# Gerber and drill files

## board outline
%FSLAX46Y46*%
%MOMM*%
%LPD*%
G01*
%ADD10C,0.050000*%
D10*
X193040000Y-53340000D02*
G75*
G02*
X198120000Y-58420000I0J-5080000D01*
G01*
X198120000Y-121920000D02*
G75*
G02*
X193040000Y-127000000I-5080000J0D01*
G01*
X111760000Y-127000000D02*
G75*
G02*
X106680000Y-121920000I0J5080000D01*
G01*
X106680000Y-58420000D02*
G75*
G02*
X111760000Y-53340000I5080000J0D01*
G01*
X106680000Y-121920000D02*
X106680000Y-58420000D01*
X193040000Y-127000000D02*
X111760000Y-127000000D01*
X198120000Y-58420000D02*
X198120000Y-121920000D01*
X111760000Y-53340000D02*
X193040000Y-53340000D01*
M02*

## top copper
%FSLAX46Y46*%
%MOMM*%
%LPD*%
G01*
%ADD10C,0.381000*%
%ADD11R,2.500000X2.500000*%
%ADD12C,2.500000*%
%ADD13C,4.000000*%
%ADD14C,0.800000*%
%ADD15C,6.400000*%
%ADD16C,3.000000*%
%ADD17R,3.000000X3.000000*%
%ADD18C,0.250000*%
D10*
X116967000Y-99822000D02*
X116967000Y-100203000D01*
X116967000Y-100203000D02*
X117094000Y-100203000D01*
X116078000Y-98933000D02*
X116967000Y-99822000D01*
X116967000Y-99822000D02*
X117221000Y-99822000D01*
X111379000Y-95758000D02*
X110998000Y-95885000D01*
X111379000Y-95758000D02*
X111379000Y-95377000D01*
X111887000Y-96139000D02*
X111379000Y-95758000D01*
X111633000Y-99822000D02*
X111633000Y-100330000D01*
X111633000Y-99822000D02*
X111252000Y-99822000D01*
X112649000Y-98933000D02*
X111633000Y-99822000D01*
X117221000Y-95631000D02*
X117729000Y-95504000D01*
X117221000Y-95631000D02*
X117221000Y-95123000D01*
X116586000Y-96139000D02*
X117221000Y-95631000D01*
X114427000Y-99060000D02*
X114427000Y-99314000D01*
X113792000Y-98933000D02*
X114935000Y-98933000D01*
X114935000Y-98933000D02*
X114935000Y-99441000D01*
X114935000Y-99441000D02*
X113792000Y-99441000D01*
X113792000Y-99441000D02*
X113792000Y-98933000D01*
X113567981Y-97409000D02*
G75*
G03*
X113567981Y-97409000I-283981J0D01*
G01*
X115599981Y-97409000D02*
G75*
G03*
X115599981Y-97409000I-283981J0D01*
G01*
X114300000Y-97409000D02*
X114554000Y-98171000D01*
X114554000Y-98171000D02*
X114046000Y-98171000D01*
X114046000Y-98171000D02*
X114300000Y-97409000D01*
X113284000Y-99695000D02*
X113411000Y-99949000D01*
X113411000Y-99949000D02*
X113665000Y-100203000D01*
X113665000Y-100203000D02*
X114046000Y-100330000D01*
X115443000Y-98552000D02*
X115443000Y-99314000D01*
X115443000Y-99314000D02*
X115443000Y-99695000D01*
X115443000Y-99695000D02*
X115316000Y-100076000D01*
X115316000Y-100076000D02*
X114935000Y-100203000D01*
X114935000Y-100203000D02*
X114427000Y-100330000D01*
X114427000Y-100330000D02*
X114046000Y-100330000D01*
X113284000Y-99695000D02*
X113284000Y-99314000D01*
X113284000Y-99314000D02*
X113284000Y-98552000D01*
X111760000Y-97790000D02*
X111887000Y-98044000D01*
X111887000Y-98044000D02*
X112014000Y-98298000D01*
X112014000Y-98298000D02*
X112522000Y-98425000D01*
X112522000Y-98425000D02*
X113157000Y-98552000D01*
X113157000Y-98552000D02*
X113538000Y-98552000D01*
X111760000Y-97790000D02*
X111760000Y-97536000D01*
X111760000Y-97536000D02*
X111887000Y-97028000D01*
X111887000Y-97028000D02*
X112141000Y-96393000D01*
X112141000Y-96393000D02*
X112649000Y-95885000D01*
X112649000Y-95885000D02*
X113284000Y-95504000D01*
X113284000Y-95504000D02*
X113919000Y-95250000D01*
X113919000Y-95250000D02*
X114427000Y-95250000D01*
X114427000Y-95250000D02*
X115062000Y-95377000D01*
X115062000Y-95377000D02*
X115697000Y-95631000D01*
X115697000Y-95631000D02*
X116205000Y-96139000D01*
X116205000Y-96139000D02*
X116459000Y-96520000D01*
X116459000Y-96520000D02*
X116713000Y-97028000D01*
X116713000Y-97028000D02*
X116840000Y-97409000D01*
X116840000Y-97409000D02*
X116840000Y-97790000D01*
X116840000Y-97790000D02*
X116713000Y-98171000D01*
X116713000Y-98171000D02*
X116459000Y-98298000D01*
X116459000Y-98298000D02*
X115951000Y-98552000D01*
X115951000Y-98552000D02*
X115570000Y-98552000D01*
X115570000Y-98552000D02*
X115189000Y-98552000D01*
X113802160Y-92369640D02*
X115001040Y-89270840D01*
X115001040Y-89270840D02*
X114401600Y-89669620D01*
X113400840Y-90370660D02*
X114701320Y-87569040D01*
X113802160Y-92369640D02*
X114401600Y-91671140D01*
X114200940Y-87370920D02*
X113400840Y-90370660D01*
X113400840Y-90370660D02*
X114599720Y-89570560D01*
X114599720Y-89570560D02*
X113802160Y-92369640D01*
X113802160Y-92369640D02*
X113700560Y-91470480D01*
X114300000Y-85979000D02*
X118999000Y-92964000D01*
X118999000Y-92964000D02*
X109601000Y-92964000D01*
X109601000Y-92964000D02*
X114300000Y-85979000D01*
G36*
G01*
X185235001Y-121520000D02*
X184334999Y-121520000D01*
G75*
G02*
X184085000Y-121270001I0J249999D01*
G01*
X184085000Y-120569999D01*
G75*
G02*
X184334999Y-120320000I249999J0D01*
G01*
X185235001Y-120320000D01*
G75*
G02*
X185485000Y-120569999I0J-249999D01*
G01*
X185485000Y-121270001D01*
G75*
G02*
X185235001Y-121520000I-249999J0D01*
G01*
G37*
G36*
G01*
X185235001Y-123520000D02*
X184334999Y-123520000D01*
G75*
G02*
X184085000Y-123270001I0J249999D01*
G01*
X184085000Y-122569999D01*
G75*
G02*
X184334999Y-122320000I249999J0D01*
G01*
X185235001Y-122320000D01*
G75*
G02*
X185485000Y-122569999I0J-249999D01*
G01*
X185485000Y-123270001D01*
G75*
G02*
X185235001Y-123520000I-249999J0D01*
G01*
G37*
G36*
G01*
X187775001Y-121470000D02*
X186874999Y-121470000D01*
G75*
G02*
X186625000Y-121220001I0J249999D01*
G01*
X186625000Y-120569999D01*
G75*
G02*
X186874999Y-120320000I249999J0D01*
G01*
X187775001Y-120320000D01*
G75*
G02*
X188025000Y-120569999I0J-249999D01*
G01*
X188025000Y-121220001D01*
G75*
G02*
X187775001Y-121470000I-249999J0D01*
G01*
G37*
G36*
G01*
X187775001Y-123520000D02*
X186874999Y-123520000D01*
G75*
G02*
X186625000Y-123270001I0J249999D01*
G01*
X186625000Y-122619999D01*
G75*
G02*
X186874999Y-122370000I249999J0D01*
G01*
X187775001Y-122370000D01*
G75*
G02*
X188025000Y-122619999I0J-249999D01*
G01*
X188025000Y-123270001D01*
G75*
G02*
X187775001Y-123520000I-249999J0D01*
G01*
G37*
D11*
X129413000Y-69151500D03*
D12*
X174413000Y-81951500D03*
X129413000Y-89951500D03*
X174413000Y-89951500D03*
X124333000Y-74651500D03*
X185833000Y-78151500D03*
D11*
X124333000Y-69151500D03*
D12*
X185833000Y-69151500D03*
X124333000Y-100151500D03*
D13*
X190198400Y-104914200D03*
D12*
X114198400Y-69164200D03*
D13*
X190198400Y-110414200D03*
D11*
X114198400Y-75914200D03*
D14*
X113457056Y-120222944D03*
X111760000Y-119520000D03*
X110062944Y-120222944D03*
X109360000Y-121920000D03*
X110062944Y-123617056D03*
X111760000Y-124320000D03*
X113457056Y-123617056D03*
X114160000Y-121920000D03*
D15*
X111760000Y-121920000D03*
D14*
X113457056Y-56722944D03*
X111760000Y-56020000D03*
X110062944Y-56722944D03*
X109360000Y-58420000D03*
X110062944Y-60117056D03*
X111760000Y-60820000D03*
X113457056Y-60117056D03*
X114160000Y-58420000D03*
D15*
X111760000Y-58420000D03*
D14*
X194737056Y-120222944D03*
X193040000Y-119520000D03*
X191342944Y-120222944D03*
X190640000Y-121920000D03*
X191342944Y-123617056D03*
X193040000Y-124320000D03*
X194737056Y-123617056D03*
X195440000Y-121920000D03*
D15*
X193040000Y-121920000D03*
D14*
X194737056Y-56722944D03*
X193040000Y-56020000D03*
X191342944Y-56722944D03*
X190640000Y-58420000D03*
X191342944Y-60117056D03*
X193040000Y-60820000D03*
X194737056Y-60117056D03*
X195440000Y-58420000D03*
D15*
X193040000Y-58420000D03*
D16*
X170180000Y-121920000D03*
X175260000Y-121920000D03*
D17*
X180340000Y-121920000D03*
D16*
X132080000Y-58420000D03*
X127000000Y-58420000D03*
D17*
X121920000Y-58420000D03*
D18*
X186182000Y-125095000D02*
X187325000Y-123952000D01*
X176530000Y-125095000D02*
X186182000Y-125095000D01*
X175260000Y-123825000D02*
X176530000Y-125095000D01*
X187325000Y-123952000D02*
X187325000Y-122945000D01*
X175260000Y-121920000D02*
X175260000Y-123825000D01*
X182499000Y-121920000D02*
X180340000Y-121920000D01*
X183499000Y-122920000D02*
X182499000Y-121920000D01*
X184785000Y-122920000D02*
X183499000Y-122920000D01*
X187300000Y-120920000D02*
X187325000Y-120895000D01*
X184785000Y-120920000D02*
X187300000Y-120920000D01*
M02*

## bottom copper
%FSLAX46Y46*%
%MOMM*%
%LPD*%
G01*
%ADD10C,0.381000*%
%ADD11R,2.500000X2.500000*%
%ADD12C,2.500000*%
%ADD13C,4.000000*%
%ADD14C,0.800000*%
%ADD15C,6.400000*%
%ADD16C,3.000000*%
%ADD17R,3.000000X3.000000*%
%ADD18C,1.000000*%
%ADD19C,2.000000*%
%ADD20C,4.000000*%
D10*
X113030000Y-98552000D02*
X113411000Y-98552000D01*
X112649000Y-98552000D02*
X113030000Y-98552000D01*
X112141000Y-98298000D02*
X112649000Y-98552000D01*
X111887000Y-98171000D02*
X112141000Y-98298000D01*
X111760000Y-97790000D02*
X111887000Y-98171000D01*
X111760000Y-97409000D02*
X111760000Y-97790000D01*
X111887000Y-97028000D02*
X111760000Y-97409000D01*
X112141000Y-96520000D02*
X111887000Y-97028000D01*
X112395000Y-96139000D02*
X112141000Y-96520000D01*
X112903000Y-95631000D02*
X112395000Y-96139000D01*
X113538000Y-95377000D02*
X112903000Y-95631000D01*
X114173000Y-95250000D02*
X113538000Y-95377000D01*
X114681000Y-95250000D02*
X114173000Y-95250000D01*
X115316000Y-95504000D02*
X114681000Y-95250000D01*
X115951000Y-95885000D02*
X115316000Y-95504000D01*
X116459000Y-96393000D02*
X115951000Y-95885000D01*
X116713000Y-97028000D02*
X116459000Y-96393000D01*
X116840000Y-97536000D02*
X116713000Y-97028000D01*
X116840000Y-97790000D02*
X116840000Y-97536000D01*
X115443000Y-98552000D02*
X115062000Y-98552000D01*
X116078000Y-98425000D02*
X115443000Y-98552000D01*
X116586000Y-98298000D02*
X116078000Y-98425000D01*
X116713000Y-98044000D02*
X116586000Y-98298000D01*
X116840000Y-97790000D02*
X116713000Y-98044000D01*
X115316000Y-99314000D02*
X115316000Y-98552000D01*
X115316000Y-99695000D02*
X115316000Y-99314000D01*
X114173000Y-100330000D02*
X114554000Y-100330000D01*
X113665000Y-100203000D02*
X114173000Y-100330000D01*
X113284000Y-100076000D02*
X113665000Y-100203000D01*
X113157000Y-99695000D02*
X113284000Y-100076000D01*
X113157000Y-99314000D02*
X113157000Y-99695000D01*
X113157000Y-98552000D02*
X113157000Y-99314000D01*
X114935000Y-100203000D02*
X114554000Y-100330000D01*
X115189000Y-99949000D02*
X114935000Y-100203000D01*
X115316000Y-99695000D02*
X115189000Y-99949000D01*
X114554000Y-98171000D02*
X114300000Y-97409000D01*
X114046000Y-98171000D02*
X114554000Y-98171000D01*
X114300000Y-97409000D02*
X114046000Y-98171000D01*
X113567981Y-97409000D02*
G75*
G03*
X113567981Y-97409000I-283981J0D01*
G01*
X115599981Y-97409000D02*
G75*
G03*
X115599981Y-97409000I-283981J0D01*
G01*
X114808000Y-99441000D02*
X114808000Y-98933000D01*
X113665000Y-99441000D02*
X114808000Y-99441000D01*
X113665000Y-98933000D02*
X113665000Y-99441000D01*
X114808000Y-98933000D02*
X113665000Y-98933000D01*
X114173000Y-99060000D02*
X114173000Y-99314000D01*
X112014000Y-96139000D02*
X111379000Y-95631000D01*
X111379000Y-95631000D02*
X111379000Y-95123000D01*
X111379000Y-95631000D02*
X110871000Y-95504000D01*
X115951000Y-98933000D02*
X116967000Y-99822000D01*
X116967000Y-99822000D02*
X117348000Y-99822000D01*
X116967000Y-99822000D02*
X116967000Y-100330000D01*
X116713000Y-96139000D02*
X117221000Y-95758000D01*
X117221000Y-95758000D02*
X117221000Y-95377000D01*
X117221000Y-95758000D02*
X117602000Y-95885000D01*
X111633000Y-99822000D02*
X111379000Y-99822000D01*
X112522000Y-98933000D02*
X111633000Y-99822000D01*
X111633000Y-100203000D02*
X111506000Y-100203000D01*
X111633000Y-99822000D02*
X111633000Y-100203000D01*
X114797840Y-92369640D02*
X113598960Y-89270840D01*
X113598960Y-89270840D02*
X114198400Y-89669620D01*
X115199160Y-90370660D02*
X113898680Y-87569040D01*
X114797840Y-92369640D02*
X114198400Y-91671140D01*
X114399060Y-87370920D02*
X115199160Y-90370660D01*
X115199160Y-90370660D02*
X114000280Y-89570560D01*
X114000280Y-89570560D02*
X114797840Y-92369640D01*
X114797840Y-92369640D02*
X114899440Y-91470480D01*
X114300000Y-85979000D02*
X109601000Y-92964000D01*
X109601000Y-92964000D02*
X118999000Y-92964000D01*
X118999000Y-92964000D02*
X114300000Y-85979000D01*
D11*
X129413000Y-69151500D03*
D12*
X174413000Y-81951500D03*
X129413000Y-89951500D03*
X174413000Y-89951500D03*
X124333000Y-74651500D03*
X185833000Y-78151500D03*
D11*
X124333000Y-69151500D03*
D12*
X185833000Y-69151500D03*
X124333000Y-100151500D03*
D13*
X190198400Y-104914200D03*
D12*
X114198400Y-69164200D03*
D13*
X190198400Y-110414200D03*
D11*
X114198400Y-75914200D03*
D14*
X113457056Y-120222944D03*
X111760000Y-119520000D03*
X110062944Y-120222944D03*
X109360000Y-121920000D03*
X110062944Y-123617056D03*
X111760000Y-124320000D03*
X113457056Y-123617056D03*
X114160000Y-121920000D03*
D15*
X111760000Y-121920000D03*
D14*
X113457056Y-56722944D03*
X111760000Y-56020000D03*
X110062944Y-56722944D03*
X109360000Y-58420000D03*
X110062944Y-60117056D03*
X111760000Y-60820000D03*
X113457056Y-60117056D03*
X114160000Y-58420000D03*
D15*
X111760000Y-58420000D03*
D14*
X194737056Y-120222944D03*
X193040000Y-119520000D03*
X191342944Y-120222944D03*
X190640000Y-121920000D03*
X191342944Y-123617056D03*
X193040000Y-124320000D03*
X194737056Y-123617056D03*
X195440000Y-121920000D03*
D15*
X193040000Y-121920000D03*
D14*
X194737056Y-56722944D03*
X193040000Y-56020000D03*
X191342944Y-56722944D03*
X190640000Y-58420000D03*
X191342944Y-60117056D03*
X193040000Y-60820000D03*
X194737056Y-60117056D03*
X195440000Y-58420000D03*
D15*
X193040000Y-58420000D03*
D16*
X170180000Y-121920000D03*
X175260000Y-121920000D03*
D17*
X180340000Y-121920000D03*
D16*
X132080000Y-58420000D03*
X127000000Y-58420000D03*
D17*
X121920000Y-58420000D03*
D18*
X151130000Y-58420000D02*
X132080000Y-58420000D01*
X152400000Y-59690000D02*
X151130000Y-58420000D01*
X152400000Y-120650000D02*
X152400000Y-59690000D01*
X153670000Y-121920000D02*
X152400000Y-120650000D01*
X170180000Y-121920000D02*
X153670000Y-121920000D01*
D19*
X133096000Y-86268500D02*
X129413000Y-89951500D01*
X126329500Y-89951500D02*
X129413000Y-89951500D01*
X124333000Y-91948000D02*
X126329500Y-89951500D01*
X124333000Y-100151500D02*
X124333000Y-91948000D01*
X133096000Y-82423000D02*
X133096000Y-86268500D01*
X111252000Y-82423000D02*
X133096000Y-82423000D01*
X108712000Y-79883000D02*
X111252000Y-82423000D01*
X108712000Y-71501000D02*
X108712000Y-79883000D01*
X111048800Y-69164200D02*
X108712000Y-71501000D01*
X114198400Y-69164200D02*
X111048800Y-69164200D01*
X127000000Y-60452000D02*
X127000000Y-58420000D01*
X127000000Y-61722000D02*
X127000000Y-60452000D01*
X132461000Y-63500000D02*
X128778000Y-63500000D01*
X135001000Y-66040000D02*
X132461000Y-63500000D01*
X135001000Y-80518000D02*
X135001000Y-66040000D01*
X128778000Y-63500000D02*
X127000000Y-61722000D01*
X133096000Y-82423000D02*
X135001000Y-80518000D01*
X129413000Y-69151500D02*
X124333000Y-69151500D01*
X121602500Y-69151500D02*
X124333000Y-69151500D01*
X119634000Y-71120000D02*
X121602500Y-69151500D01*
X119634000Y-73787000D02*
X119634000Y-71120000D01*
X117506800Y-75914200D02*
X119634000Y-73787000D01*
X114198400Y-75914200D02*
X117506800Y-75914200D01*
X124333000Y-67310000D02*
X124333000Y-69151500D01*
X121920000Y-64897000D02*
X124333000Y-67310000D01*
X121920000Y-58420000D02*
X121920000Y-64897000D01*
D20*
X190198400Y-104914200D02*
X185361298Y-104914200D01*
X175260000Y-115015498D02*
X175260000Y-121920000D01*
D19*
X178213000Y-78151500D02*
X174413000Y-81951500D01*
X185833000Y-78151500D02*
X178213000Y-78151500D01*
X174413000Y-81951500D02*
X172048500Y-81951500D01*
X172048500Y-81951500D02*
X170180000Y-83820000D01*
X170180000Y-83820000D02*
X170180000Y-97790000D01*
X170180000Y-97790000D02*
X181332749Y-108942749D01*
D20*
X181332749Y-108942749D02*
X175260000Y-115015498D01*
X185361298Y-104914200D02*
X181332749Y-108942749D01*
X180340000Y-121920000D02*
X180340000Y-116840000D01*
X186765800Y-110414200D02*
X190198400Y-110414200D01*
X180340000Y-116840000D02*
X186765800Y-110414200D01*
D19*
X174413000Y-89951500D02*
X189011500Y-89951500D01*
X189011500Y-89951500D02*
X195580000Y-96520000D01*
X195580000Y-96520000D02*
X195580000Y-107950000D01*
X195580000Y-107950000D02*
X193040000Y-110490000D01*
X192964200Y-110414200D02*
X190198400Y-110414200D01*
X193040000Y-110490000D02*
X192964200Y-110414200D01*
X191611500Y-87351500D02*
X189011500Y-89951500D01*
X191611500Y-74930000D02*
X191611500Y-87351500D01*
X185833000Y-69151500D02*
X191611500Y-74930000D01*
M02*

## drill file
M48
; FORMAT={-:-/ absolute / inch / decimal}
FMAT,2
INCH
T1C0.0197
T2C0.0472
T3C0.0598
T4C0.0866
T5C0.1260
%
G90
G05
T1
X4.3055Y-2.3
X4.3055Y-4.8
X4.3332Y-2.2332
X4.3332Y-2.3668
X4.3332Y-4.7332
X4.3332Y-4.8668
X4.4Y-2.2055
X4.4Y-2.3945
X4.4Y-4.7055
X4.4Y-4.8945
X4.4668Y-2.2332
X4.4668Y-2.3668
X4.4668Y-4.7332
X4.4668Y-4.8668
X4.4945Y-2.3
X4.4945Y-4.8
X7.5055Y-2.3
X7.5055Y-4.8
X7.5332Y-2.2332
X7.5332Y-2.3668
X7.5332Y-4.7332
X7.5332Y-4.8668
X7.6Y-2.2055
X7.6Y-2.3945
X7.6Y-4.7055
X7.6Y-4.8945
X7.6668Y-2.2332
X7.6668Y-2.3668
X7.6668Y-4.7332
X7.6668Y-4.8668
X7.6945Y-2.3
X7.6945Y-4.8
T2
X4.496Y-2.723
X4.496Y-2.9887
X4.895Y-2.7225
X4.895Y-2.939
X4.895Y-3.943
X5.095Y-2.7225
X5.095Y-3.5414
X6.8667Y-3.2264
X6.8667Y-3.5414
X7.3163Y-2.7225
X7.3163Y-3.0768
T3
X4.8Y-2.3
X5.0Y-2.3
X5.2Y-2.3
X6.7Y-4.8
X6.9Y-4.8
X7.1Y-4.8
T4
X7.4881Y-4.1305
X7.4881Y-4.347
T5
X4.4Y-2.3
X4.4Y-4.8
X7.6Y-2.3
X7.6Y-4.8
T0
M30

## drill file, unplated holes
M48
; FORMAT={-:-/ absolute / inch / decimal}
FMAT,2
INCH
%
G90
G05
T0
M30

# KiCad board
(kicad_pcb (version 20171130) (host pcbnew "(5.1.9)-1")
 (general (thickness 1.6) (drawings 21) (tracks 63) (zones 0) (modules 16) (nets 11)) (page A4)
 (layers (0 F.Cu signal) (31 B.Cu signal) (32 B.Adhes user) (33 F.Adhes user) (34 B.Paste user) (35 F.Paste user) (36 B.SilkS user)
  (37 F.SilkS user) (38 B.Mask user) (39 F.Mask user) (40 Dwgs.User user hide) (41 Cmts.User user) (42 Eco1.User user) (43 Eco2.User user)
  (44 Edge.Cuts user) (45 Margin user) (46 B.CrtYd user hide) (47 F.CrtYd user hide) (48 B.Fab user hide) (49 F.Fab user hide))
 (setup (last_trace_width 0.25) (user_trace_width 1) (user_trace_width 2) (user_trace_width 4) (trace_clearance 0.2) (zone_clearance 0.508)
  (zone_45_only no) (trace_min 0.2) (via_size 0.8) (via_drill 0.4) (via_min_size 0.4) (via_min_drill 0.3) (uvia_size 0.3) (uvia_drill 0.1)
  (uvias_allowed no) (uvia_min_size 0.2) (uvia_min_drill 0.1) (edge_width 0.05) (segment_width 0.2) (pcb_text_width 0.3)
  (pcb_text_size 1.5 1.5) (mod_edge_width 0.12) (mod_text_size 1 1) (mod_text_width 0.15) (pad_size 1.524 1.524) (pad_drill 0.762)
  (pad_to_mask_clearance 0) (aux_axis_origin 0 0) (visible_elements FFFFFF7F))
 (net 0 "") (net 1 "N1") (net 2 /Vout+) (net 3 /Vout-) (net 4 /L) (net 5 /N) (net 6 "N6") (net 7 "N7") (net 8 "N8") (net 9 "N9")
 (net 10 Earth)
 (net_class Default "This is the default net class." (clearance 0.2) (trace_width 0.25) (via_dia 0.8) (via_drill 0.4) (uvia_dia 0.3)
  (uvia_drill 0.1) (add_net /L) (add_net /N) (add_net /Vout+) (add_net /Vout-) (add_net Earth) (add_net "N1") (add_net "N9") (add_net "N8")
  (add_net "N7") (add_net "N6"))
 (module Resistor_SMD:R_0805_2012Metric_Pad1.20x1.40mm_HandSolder (layer F.Cu) (at 184.785 121.92 90)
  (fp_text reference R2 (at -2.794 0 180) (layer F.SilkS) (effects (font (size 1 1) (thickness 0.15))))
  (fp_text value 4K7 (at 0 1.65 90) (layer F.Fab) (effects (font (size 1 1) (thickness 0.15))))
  (pad 2 smd roundrect (at 1 0 90) (size 1.2 1.4) (layers F.Cu F.Paste F.Mask) (roundrect_rratio 0.2083325) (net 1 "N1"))
  (pad 1 smd roundrect (at -1 0 90) (size 1.2 1.4) (layers F.Cu F.Paste F.Mask) (roundrect_rratio 0.2083325) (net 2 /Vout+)))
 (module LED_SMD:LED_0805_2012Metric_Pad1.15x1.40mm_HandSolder (layer F.Cu) (at 187.325 121.92 90)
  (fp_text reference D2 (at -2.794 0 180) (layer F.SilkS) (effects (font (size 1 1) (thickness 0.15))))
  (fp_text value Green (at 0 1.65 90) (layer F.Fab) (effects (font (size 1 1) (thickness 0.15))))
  (pad 2 smd roundrect (at 1.025 0 90) (size 1.15 1.4) (layers F.Cu F.Paste F.Mask) (roundrect_rratio 0.2173904347826087) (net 1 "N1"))
  (pad 1 smd roundrect (at -1.025 0 90) (size 1.15 1.4) (layers F.Cu F.Paste F.Mask) (roundrect_rratio 0.2173904347826087) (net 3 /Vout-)))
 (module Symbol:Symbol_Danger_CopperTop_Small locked (layer B.Cu) (at 114.3 97.79 180)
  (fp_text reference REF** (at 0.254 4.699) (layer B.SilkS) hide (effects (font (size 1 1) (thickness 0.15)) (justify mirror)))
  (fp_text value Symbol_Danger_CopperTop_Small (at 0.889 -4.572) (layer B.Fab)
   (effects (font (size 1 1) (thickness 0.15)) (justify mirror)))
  (fp_line (start 1.27 -0.762) (end 0.889 -0.762) (layer B.Cu) (width 0.381))
  (fp_line (start 1.651 -0.762) (end 1.27 -0.762) (layer B.Cu) (width 0.381))
  (fp_line (start 2.159 -0.508) (end 1.651 -0.762) (layer B.Cu) (width 0.381))
  (fp_line (start 2.413 -0.381) (end 2.159 -0.508) (layer B.Cu) (width 0.381))
  (fp_line (start 2.54 0) (end 2.413 -0.381) (layer B.Cu) (width 0.381))
  (fp_line (start 2.54 0.381) (end 2.54 0) (layer B.Cu) (width 0.381))
  (fp_line (start 2.413 0.762) (end 2.54 0.381) (layer B.Cu) (width 0.381))
  (fp_line (start 2.159 1.27) (end 2.413 0.762) (layer B.Cu) (width 0.381))
  (fp_line (start 1.905 1.651) (end 2.159 1.27) (layer B.Cu) (width 0.381))
  (fp_line (start 1.397 2.159) (end 1.905 1.651) (layer B.Cu) (width 0.381))
  (fp_line (start 0.762 2.413) (end 1.397 2.159) (layer B.Cu) (width 0.381))
  (fp_line (start 0.127 2.54) (end 0.762 2.413) (layer B.Cu) (width 0.381))
  (fp_line (start -0.381 2.54) (end 0.127 2.54) (layer B.Cu) (width 0.381))
  (fp_line (start -1.016 2.286) (end -0.381 2.54) (layer B.Cu) (width 0.381))
  (fp_line (start -1.651 1.905) (end -1.016 2.286) (layer B.Cu) (width 0.381))
  (fp_line (start -2.159 1.397) (end -1.651 1.905) (layer B.Cu) (width 0.381))
  (fp_line (start -2.413 0.762) (end -2.159 1.397) (layer B.Cu) (width 0.381))
  (fp_line (start -2.54 0.254) (end -2.413 0.762) (layer B.Cu) (width 0.381))
  (fp_line (start -2.54 0) (end -2.54 0.254) (layer B.Cu) (width 0.381))
  (fp_line (start -1.143 -0.762) (end -0.762 -0.762) (layer B.Cu) (width 0.381))
  (fp_line (start -1.778 -0.635) (end -1.143 -0.762) (layer B.Cu) (width 0.381))
  (fp_line (start -2.286 -0.508) (end -1.778 -0.635) (layer B.Cu) (width 0.381))
  (fp_line (start -2.413 -0.254) (end -2.286 -0.508) (layer B.Cu) (width 0.381))
  (fp_line (start -2.54 0) (end -2.413 -0.254) (layer B.Cu) (width 0.381))
  (fp_line (start -1.016 -1.524) (end -1.016 -0.762) (layer B.Cu) (width 0.381))
  (fp_line (start -1.016 -1.905) (end -1.016 -1.524) (layer B.Cu) (width 0.381))
  (fp_line (start 0.127 -2.54) (end -0.254 -2.54) (layer B.Cu) (width 0.381))
  (fp_line (start 0.635 -2.413) (end 0.127 -2.54) (layer B.Cu) (width 0.381))
  (fp_line (start 1.016 -2.286) (end 0.635 -2.413) (layer B.Cu) (width 0.381))
  (fp_line (start 1.143 -1.905) (end 1.016 -2.286) (layer B.Cu) (width 0.381))
  (fp_line (start 1.143 -1.524) (end 1.143 -1.905) (layer B.Cu) (width 0.381))
  (fp_line (start 1.143 -0.762) (end 1.143 -1.524) (layer B.Cu) (width 0.381))
  (fp_line (start -0.635 -2.413) (end -0.254 -2.54) (layer B.Cu) (width 0.381))
  (fp_line (start -0.889 -2.159) (end -0.635 -2.413) (layer B.Cu) (width 0.381))
  (fp_line (start -1.016 -1.905) (end -0.889 -2.159) (layer B.Cu) (width 0.381))
  (fp_line (start -0.254 -0.381) (end 0 0.381) (layer B.Cu) (width 0.381))
  (fp_line (start 0.254 -0.381) (end -0.254 -0.381) (layer B.Cu) (width 0.381))
  (fp_line (start 0 0.381) (end 0.254 -0.381) (layer B.Cu) (width 0.381))
  (fp_circle (center 1.016 0.381) (end 1.27 0.254) (layer B.Cu) (width 0.381))
  (fp_circle (center -1.016 0.381) (end -1.27 0.254) (layer B.Cu) (width 0.381))
  (fp_line (start -0.508 -1.651) (end -0.508 -1.143) (layer B.Cu) (width 0.381))
  (fp_line (start 0.635 -1.651) (end -0.508 -1.651) (layer B.Cu) (width 0.381))
  (fp_line (start 0.635 -1.143) (end 0.635 -1.651) (layer B.Cu) (width 0.381))
  (fp_line (start -0.508 -1.143) (end 0.635 -1.143) (layer B.Cu) (width 0.381))
  (fp_line (start 0.127 -1.27) (end 0.127 -1.524) (layer B.Cu) (width 0.381))
  (fp_line (start 2.286 1.651) (end 2.921 2.159) (layer B.Cu) (width 0.381))
  (fp_line (start 2.921 2.159) (end 2.921 2.667) (layer B.Cu) (width 0.381))
  (fp_line (start 2.921 2.159) (end 3.429 2.286) (layer B.Cu) (width 0.381))
  (fp_line (start -1.651 -1.143) (end -2.667 -2.032) (layer B.Cu) (width 0.381))
  (fp_line (start -2.667 -2.032) (end -3.048 -2.032) (layer B.Cu) (width 0.381))
  (fp_line (start -2.667 -2.032) (end -2.667 -2.54) (layer B.Cu) (width 0.381))
  (fp_line (start -2.413 1.651) (end -2.921 2.032) (layer B.Cu) (width 0.381))
  (fp_line (start -2.921 2.032) (end -2.921 2.413) (layer B.Cu) (width 0.381))
  (fp_line (start -2.921 2.032) (end -3.302 1.905) (layer B.Cu) (width 0.381))
  (fp_line (start 2.667 -2.032) (end 2.921 -2.032) (layer B.Cu) (width 0.381))
  (fp_line (start 1.778 -1.143) (end 2.667 -2.032) (layer B.Cu) (width 0.381))
  (fp_line (start 2.667 -2.413) (end 2.794 -2.413) (layer B.Cu) (width 0.381))
  (fp_line (start 2.667 -2.032) (end 2.667 -2.413) (layer B.Cu) (width 0.381)))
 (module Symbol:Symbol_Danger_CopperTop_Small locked (layer F.Cu) (at 114.3 97.79)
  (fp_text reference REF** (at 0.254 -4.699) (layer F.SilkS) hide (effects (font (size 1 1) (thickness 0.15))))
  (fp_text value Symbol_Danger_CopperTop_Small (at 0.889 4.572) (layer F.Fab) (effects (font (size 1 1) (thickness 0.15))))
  (fp_line (start 2.667 2.032) (end 2.667 2.413) (layer F.Cu) (width 0.381))
  (fp_line (start 2.667 2.413) (end 2.794 2.413) (layer F.Cu) (width 0.381))
  (fp_line (start 1.778 1.143) (end 2.667 2.032) (layer F.Cu) (width 0.381))
  (fp_line (start 2.667 2.032) (end 2.921 2.032) (layer F.Cu) (width 0.381))
  (fp_line (start -2.921 -2.032) (end -3.302 -1.905) (layer F.Cu) (width 0.381))
  (fp_line (start -2.921 -2.032) (end -2.921 -2.413) (layer F.Cu) (width 0.381))
  (fp_line (start -2.413 -1.651) (end -2.921 -2.032) (layer F.Cu) (width 0.381))
  (fp_line (start -2.667 2.032) (end -2.667 2.54) (layer F.Cu) (width 0.381))
  (fp_line (start -2.667 2.032) (end -3.048 2.032) (layer F.Cu) (width 0.381))
  (fp_line (start -1.651 1.143) (end -2.667 2.032) (layer F.Cu) (width 0.381))
  (fp_line (start 2.921 -2.159) (end 3.429 -2.286) (layer F.Cu) (width 0.381))
  (fp_line (start 2.921 -2.159) (end 2.921 -2.667) (layer F.Cu) (width 0.381))
  (fp_line (start 2.286 -1.651) (end 2.921 -2.159) (layer F.Cu) (width 0.381))
  (fp_line (start 0.127 1.27) (end 0.127 1.524) (layer F.Cu) (width 0.381))
  (fp_line (start -0.508 1.143) (end 0.635 1.143) (layer F.Cu) (width 0.381))
  (fp_line (start 0.635 1.143) (end 0.635 1.651) (layer F.Cu) (width 0.381))
  (fp_line (start 0.635 1.651) (end -0.508 1.651) (layer F.Cu) (width 0.381))
  (fp_line (start -0.508 1.651) (end -0.508 1.143) (layer F.Cu) (width 0.381))
  (fp_circle (center -1.016 -0.381) (end -1.27 -0.254) (layer F.Cu) (width 0.381))
  (fp_circle (center 1.016 -0.381) (end 1.27 -0.254) (layer F.Cu) (width 0.381))
  (fp_line (start 0 -0.381) (end 0.254 0.381) (layer F.Cu) (width 0.381))
  (fp_line (start 0.254 0.381) (end -0.254 0.381) (layer F.Cu) (width 0.381))
  (fp_line (start -0.254 0.381) (end 0 -0.381) (layer F.Cu) (width 0.381))
  (fp_line (start -1.016 1.905) (end -0.889 2.159) (layer F.Cu) (width 0.381))
  (fp_line (start -0.889 2.159) (end -0.635 2.413) (layer F.Cu) (width 0.381))
  (fp_line (start -0.635 2.413) (end -0.254 2.54) (layer F.Cu) (width 0.381))
  (fp_line (start 1.143 0.762) (end 1.143 1.524) (layer F.Cu) (width 0.381))
  (fp_line (start 1.143 1.524) (end 1.143 1.905) (layer F.Cu) (width 0.381))
  (fp_line (start 1.143 1.905) (end 1.016 2.286) (layer F.Cu) (width 0.381))
  (fp_line (start 1.016 2.286) (end 0.635 2.413) (layer F.Cu) (width 0.381))
  (fp_line (start 0.635 2.413) (end 0.127 2.54) (layer F.Cu) (width 0.381))
  (fp_line (start 0.127 2.54) (end -0.254 2.54) (layer F.Cu) (width 0.381))
  (fp_line (start -1.016 1.905) (end -1.016 1.524) (layer F.Cu) (width 0.381))
  (fp_line (start -1.016 1.524) (end -1.016 0.762) (layer F.Cu) (width 0.381))
  (fp_line (start -2.54 0) (end -2.413 0.254) (layer F.Cu) (width 0.381))
  (fp_line (start -2.413 0.254) (end -2.286 0.508) (layer F.Cu) (width 0.381))
  (fp_line (start -2.286 0.508) (end -1.778 0.635) (layer F.Cu) (width 0.381))
  (fp_line (start -1.778 0.635) (end -1.143 0.762) (layer F.Cu) (width 0.381))
  (fp_line (start -1.143 0.762) (end -0.762 0.762) (layer F.Cu) (width 0.381))
  (fp_line (start -2.54 0) (end -2.54 -0.254) (layer F.Cu) (width 0.381))
  (fp_line (start -2.54 -0.254) (end -2.413 -0.762) (layer F.Cu) (width 0.381))
  (fp_line (start -2.413 -0.762) (end -2.159 -1.397) (layer F.Cu) (width 0.381))
  (fp_line (start -2.159 -1.397) (end -1.651 -1.905) (layer F.Cu) (width 0.381))
  (fp_line (start -1.651 -1.905) (end -1.016 -2.286) (layer F.Cu) (width 0.381))
  (fp_line (start -1.016 -2.286) (end -0.381 -2.54) (layer F.Cu) (width 0.381))
  (fp_line (start -0.381 -2.54) (end 0.127 -2.54) (layer F.Cu) (width 0.381))
  (fp_line (start 0.127 -2.54) (end 0.762 -2.413) (layer F.Cu) (width 0.381))
  (fp_line (start 0.762 -2.413) (end 1.397 -2.159) (layer F.Cu) (width 0.381))
  (fp_line (start 1.397 -2.159) (end 1.905 -1.651) (layer F.Cu) (width 0.381))
  (fp_line (start 1.905 -1.651) (end 2.159 -1.27) (layer F.Cu) (width 0.381))
  (fp_line (start 2.159 -1.27) (end 2.413 -0.762) (layer F.Cu) (width 0.381))
  (fp_line (start 2.413 -0.762) (end 2.54 -0.381) (layer F.Cu) (width 0.381))
  (fp_line (start 2.54 -0.381) (end 2.54 0) (layer F.Cu) (width 0.381))
  (fp_line (start 2.54 0) (end 2.413 0.381) (layer F.Cu) (width 0.381))
  (fp_line (start 2.413 0.381) (end 2.159 0.508) (layer F.Cu) (width 0.381))
  (fp_line (start 2.159 0.508) (end 1.651 0.762) (layer F.Cu) (width 0.381))
  (fp_line (start 1.651 0.762) (end 1.27 0.762) (layer F.Cu) (width 0.381))
  (fp_line (start 1.27 0.762) (end 0.889 0.762) (layer F.Cu) (width 0.381)))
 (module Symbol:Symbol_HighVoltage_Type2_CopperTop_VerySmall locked (layer B.Cu) (at 114.3 90.17 180)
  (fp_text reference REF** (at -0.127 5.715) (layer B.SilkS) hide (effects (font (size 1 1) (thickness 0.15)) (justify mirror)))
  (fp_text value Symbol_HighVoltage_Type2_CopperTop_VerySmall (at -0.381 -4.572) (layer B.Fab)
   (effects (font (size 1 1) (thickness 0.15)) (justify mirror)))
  (fp_line (start -0.49784 -2.19964) (end 0.70104 0.89916) (layer B.Cu) (width 0.381))
  (fp_line (start 0.70104 0.89916) (end 0.1016 0.50038) (layer B.Cu) (width 0.381))
  (fp_line (start -0.89916 -0.20066) (end 0.40132 2.60096) (layer B.Cu) (width 0.381))
  (fp_line (start -0.49784 -2.19964) (end 0.1016 -1.50114) (layer B.Cu) (width 0.381))
  (fp_line (start -0.09906 2.79908) (end -0.89916 -0.20066) (layer B.Cu) (width 0.381))
  (fp_line (start -0.89916 -0.20066) (end 0.29972 0.59944) (layer B.Cu) (width 0.381))
  (fp_line (start 0.29972 0.59944) (end -0.49784 -2.19964) (layer B.Cu) (width 0.381))
  (fp_line (start -0.49784 -2.19964) (end -0.59944 -1.30048) (layer B.Cu) (width 0.381))
  (fp_line (start 0 4.191) (end 4.699 -2.794) (layer B.Cu) (width 0.381))
  (fp_line (start 4.699 -2.794) (end -4.699 -2.794) (layer B.Cu) (width 0.381))
  (fp_line (start -4.699 -2.794) (end 0 4.191) (layer B.Cu) (width 0.381)))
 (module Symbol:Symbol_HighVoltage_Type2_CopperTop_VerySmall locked (layer F.Cu) (at 114.3 90.17)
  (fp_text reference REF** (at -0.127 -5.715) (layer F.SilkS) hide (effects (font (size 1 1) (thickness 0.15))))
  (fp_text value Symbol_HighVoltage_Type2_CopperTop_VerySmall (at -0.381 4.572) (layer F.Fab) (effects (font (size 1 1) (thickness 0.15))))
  (fp_line (start -0.49784 2.19964) (end 0.70104 -0.89916) (layer F.Cu) (width 0.381))
  (fp_line (start 0.70104 -0.89916) (end 0.1016 -0.50038) (layer F.Cu) (width 0.381))
  (fp_line (start -0.89916 0.20066) (end 0.40132 -2.60096) (layer F.Cu) (width 0.381))
  (fp_line (start -0.49784 2.19964) (end 0.1016 1.50114) (layer F.Cu) (width 0.381))
  (fp_line (start -0.09906 -2.79908) (end -0.89916 0.20066) (layer F.Cu) (width 0.381))
  (fp_line (start -0.89916 0.20066) (end 0.29972 -0.59944) (layer F.Cu) (width 0.381))
  (fp_line (start 0.29972 -0.59944) (end -0.49784 2.19964) (layer F.Cu) (width 0.381))
  (fp_line (start -0.49784 2.19964) (end -0.59944 1.30048) (layer F.Cu) (width 0.381))
  (fp_line (start 0 -4.191) (end 4.699 2.794) (layer F.Cu) (width 0.381))
  (fp_line (start 4.699 2.794) (end -4.699 2.794) (layer F.Cu) (width 0.381))
  (fp_line (start -4.699 2.794) (end 0 -4.191) (layer F.Cu) (width 0.381)))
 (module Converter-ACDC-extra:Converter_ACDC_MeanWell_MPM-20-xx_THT (layer F.Cu) (at 152.213 79.5515)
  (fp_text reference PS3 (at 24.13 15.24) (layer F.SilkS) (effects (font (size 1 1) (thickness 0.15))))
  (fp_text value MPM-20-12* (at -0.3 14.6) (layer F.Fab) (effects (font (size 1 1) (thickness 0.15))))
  (pad 1 thru_hole rect (at -22.8 -10.4) (size 2.5 2.5) (drill 1.2) (layers *.Cu *.Mask) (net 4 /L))
  (pad 4 thru_hole circle (at 22.2 2.4) (size 2.5 2.5) (drill 1.2) (layers *.Cu *.Mask) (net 3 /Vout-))
  (pad 2 thru_hole circle (at -22.8 10.4) (size 2.5 2.5) (drill 1.2) (layers *.Cu *.Mask) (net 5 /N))
  (pad 3 thru_hole circle (at 22.2 10.4) (size 2.5 2.5) (drill 1.2) (layers *.Cu *.Mask) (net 2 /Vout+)))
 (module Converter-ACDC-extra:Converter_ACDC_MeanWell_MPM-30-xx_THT (layer F.Cu) (at 155.083 84.1515)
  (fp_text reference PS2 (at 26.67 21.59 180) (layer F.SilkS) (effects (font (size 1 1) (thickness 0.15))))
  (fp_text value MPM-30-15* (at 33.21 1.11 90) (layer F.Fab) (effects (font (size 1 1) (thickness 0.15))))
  (pad ~ thru_hole circle (at -30.75 -9.5) (size 2.5 2.5) (drill 1.2) (layers *.Cu *.Mask))
  (pad 4 thru_hole circle (at 30.75 -6 90) (size 2.5 2.5) (drill 1.2) (layers *.Cu *.Mask) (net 3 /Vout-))
  (pad 1 thru_hole rect (at -30.75 -15) (size 2.5 2.5) (drill 1.2) (layers *.Cu *.Mask) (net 4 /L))
  (pad 3 thru_hole circle (at 30.75 -15) (size 2.5 2.5) (drill 1.2) (layers *.Cu *.Mask) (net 2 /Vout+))
  (pad 2 thru_hole circle (at -30.75 16) (size 2.5 2.5) (drill 1.2) (layers *.Cu *.Mask) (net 5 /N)))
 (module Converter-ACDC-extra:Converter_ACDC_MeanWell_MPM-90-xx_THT (layer F.Cu) (at 152.4 90.17)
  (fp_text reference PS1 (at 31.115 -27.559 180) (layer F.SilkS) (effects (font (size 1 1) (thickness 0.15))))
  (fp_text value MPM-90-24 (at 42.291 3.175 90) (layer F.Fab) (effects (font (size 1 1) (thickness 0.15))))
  (pad 4 thru_hole circle (at 37.7984 14.7442) (size 4 4) (drill 2.2) (layers *.Cu *.Mask) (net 3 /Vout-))
  (pad 2 thru_hole circle (at -38.2016 -21.0058) (size 2.5 2.5) (drill 1.2) (layers *.Cu *.Mask) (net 5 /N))
  (pad 3 thru_hole circle (at 37.7984 20.2442) (size 4 4) (drill 2.2) (layers *.Cu *.Mask) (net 2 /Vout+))
  (pad 1 thru_hole rect (at -38.2016 -14.2558) (size 2.5 2.5) (drill 1.2) (layers *.Cu *.Mask) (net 4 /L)))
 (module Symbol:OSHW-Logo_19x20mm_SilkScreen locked (layer B.Cu) (at 152.4 109.22 180)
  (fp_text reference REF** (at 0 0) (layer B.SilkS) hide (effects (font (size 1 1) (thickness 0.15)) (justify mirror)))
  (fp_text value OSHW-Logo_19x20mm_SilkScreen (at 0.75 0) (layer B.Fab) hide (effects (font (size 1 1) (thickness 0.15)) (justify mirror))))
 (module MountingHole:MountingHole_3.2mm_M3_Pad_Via (layer F.Cu) (at 111.76 121.92)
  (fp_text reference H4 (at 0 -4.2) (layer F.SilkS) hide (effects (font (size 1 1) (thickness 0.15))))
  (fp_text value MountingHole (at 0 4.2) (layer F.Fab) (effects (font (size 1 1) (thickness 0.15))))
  (pad 1 thru_hole circle (at 1.697056 -1.697056) (size 0.8 0.8) (drill 0.5) (layers *.Cu *.Mask) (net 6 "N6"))
  (pad 1 thru_hole circle (at 0 -2.4) (size 0.8 0.8) (drill 0.5) (layers *.Cu *.Mask) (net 6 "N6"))
  (pad 1 thru_hole circle (at -1.697056 -1.697056) (size 0.8 0.8) (drill 0.5) (layers *.Cu *.Mask) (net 6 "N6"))
  (pad 1 thru_hole circle (at -2.4 0) (size 0.8 0.8) (drill 0.5) (layers *.Cu *.Mask) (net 6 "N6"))
  (pad 1 thru_hole circle (at -1.697056 1.697056) (size 0.8 0.8) (drill 0.5) (layers *.Cu *.Mask) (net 6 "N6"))
  (pad 1 thru_hole circle (at 0 2.4) (size 0.8 0.8) (drill 0.5) (layers *.Cu *.Mask) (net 6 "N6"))
  (pad 1 thru_hole circle (at 1.697056 1.697056) (size 0.8 0.8) (drill 0.5) (layers *.Cu *.Mask) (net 6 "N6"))
  (pad 1 thru_hole circle (at 2.4 0) (size 0.8 0.8) (drill 0.5) (layers *.Cu *.Mask) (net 6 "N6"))
  (pad 1 thru_hole circle (at 0 0) (size 6.4 6.4) (drill 3.2) (layers *.Cu *.Mask) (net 6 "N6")))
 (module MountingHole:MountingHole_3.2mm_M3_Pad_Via (layer F.Cu) (at 111.76 58.42)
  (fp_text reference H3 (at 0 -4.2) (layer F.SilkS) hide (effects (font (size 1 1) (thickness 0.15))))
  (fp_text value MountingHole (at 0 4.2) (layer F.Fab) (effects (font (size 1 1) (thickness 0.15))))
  (pad 1 thru_hole circle (at 1.697056 -1.697056) (size 0.8 0.8) (drill 0.5) (layers *.Cu *.Mask) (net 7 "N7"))
  (pad 1 thru_hole circle (at 0 -2.4) (size 0.8 0.8) (drill 0.5) (layers *.Cu *.Mask) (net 7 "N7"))
  (pad 1 thru_hole circle (at -1.697056 -1.697056) (size 0.8 0.8) (drill 0.5) (layers *.Cu *.Mask) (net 7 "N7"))
  (pad 1 thru_hole circle (at -2.4 0) (size 0.8 0.8) (drill 0.5) (layers *.Cu *.Mask) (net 7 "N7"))
  (pad 1 thru_hole circle (at -1.697056 1.697056) (size 0.8 0.8) (drill 0.5) (layers *.Cu *.Mask) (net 7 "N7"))
  (pad 1 thru_hole circle (at 0 2.4) (size 0.8 0.8) (drill 0.5) (layers *.Cu *.Mask) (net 7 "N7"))
  (pad 1 thru_hole circle (at 1.697056 1.697056) (size 0.8 0.8) (drill 0.5) (layers *.Cu *.Mask) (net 7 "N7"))
  (pad 1 thru_hole circle (at 2.4 0) (size 0.8 0.8) (drill 0.5) (layers *.Cu *.Mask) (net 7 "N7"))
  (pad 1 thru_hole circle (at 0 0) (size 6.4 6.4) (drill 3.2) (layers *.Cu *.Mask) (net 7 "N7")))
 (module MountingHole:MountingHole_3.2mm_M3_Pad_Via (layer F.Cu) (at 193.04 121.92)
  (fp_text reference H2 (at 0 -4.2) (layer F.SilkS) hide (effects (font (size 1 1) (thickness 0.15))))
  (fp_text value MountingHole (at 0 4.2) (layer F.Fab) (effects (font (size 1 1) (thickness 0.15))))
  (pad 1 thru_hole circle (at 1.697056 -1.697056) (size 0.8 0.8) (drill 0.5) (layers *.Cu *.Mask) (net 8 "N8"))
  (pad 1 thru_hole circle (at 0 -2.4) (size 0.8 0.8) (drill 0.5) (layers *.Cu *.Mask) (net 8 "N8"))
  (pad 1 thru_hole circle (at -1.697056 -1.697056) (size 0.8 0.8) (drill 0.5) (layers *.Cu *.Mask) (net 8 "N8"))
  (pad 1 thru_hole circle (at -2.4 0) (size 0.8 0.8) (drill 0.5) (layers *.Cu *.Mask) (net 8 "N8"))
  (pad 1 thru_hole circle (at -1.697056 1.697056) (size 0.8 0.8) (drill 0.5) (layers *.Cu *.Mask) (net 8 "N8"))
  (pad 1 thru_hole circle (at 0 2.4) (size 0.8 0.8) (drill 0.5) (layers *.Cu *.Mask) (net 8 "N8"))
  (pad 1 thru_hole circle (at 1.697056 1.697056) (size 0.8 0.8) (drill 0.5) (layers *.Cu *.Mask) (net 8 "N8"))
  (pad 1 thru_hole circle (at 2.4 0) (size 0.8 0.8) (drill 0.5) (layers *.Cu *.Mask) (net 8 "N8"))
  (pad 1 thru_hole circle (at 0 0) (size 6.4 6.4) (drill 3.2) (layers *.Cu *.Mask) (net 8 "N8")))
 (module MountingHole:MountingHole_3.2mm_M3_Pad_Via (layer F.Cu) (at 193.04 58.42)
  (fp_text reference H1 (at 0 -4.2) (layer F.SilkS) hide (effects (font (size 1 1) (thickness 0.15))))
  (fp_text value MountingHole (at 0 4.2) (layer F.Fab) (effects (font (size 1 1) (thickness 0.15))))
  (pad 1 thru_hole circle (at 1.697056 -1.697056) (size 0.8 0.8) (drill 0.5) (layers *.Cu *.Mask) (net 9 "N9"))
  (pad 1 thru_hole circle (at 0 -2.4) (size 0.8 0.8) (drill 0.5) (layers *.Cu *.Mask) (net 9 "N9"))
  (pad 1 thru_hole circle (at -1.697056 -1.697056) (size 0.8 0.8) (drill 0.5) (layers *.Cu *.Mask) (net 9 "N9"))
  (pad 1 thru_hole circle (at -2.4 0) (size 0.8 0.8) (drill 0.5) (layers *.Cu *.Mask) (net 9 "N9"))
  (pad 1 thru_hole circle (at -1.697056 1.697056) (size 0.8 0.8) (drill 0.5) (layers *.Cu *.Mask) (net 9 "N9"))
  (pad 1 thru_hole circle (at 0 2.4) (size 0.8 0.8) (drill 0.5) (layers *.Cu *.Mask) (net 9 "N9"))
  (pad 1 thru_hole circle (at 1.697056 1.697056) (size 0.8 0.8) (drill 0.5) (layers *.Cu *.Mask) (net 9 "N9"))
  (pad 1 thru_hole circle (at 2.4 0) (size 0.8 0.8) (drill 0.5) (layers *.Cu *.Mask) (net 9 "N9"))
  (pad 1 thru_hole circle (at 0 0) (size 6.4 6.4) (drill 3.2) (layers *.Cu *.Mask) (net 9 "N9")))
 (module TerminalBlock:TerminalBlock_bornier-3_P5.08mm (layer F.Cu) (at 180.34 121.92 180)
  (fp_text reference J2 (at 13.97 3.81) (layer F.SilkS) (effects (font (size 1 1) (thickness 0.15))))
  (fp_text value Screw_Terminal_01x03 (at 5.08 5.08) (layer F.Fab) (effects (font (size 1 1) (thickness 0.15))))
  (pad 3 thru_hole circle (at 10.16 0 180) (size 3 3) (drill 1.52) (layers *.Cu *.Mask) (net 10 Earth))
  (pad 2 thru_hole circle (at 5.08 0 180) (size 3 3) (drill 1.52) (layers *.Cu *.Mask) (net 3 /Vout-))
  (pad 1 thru_hole rect (at 0 0 180) (size 3 3) (drill 1.52) (layers *.Cu *.Mask) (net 2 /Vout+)))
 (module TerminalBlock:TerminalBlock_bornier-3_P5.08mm (layer F.Cu) (at 121.92 58.42)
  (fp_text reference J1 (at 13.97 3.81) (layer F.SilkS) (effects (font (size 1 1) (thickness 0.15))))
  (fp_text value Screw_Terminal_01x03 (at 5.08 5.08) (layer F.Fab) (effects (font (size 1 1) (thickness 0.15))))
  (pad 3 thru_hole circle (at 10.16 0) (size 3 3) (drill 1.52) (layers *.Cu *.Mask) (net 10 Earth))
  (pad 2 thru_hole circle (at 5.08 0) (size 3 3) (drill 1.52) (layers *.Cu *.Mask) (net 5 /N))
  (pad 1 thru_hole rect (at 0 0) (size 3 3) (drill 1.52) (layers *.Cu *.Mask) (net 4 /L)))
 (gr_arc (start 193.04 58.42) (end 198.12 58.42) (angle -90) (layer Edge.Cuts) (width 0.05))
 (gr_arc (start 193.04 121.92) (end 193.04 127) (angle -90) (layer Edge.Cuts) (width 0.05))
 (gr_arc (start 111.76 121.92) (end 106.68 121.92) (angle -90) (layer Edge.Cuts) (width 0.05))
 (gr_arc (start 111.76 58.42) (end 111.76 53.34) (angle -90) (layer Edge.Cuts) (width 0.05))
 (gr_line (start 106.68 121.92) (end 106.68 58.42) (layer Edge.Cuts) (width 0.05))
 (gr_line (start 193.04 127) (end 111.76 127) (layer Edge.Cuts) (width 0.05))
 (gr_line (start 198.12 58.42) (end 198.12 121.92) (layer Edge.Cuts) (width 0.05))
 (gr_line (start 111.76 53.34) (end 193.04 53.34) (layer Edge.Cuts) (width 0.05))
 (segment (start 151.13 58.42) (end 132.08 58.42) (width 1) (layer B.Cu) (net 10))
 (segment (start 152.4 59.69) (end 151.13 58.42) (width 1) (layer B.Cu) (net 10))
 (segment (start 152.4 120.65) (end 152.4 59.69) (width 1) (layer B.Cu) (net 10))
 (segment (start 153.67 121.92) (end 152.4 120.65) (width 1) (layer B.Cu) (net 10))
 (segment (start 170.18 121.92) (end 153.67 121.92) (width 1) (layer B.Cu) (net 10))
 (segment (start 133.096 86.2685) (end 129.413 89.9515) (width 2) (layer B.Cu) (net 5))
 (segment (start 126.3295 89.9515) (end 129.413 89.9515) (width 2) (layer B.Cu) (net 5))
 (segment (start 124.333 91.948) (end 126.3295 89.9515) (width 2) (layer B.Cu) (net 5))
 (segment (start 124.333 100.1515) (end 124.333 91.948) (width 2) (layer B.Cu) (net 5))
 (segment (start 133.096 82.423) (end 133.096 86.2685) (width 2) (layer B.Cu) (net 5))
 (segment (start 111.252 82.423) (end 133.096 82.423) (width 2) (layer B.Cu) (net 5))
 (segment (start 108.712 79.883) (end 111.252 82.423) (width 2) (layer B.Cu) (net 5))
 (segment (start 108.712 71.501) (end 108.712 79.883) (width 2) (layer B.Cu) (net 5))
 (segment (start 111.0488 69.1642) (end 108.712 71.501) (width 2) (layer B.Cu) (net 5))
 (segment (start 114.1984 69.1642) (end 111.0488 69.1642) (width 2) (layer B.Cu) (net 5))
 (segment (start 127 60.452) (end 127 58.42) (width 2) (layer B.Cu) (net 5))
 (segment (start 127 61.722) (end 127 60.452) (width 2) (layer B.Cu) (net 5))
 (segment (start 132.461 63.5) (end 128.778 63.5) (width 2) (layer B.Cu) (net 5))
 (segment (start 135.001 66.04) (end 132.461 63.5) (width 2) (layer B.Cu) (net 5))
 (segment (start 135.001 80.518) (end 135.001 66.04) (width 2) (layer B.Cu) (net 5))
 (segment (start 128.778 63.5) (end 127 61.722) (width 2) (layer B.Cu) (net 5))
 (segment (start 133.096 82.423) (end 135.001 80.518) (width 2) (layer B.Cu) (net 5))
 (segment (start 129.413 69.1515) (end 124.333 69.1515) (width 2) (layer B.Cu) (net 4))
 (segment (start 121.6025 69.1515) (end 124.333 69.1515) (width 2) (layer B.Cu) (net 4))
 (segment (start 119.634 71.12) (end 121.6025 69.1515) (width 2) (layer B.Cu) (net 4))
 (segment (start 119.634 73.787) (end 119.634 71.12) (width 2) (layer B.Cu) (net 4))
 (segment (start 117.5068 75.9142) (end 119.634 73.787) (width 2) (layer B.Cu) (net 4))
 (segment (start 114.1984 75.9142) (end 117.5068 75.9142) (width 2) (layer B.Cu) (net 4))
 (segment (start 124.333 67.31) (end 124.333 69.1515) (width 2) (layer B.Cu) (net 4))
 (segment (start 121.92 64.897) (end 124.333 67.31) (width 2) (layer B.Cu) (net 4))
 (segment (start 121.92 58.42) (end 121.92 64.897) (width 2) (layer B.Cu) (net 4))
 (segment (start 190.1984 104.9142) (end 185.361298 104.9142) (width 4) (layer B.Cu) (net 3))
 (segment (start 175.26 115.015498) (end 175.26 121.92) (width 4) (layer B.Cu) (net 3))
 (segment (start 178.213 78.1515) (end 174.413 81.9515) (width 2) (layer B.Cu) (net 3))
 (segment (start 185.833 78.1515) (end 178.213 78.1515) (width 2) (layer B.Cu) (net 3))
 (segment (start 174.413 81.9515) (end 172.0485 81.9515) (width 2) (layer B.Cu) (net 3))
 (segment (start 172.0485 81.9515) (end 170.18 83.82) (width 2) (layer B.Cu) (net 3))
 (segment (start 170.18 83.82) (end 170.18 97.79) (width 2) (layer B.Cu) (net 3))
 (segment (start 170.18 97.79) (end 181.332749 108.942749) (width 2) (layer B.Cu) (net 3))
 (segment (start 181.332749 108.942749) (end 175.26 115.015498) (width 4) (layer B.Cu) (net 3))
 (segment (start 185.361298 104.9142) (end 181.332749 108.942749) (width 4) (layer B.Cu) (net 3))
 (segment (start 186.182 125.095) (end 187.325 123.952) (width 0.25) (layer F.Cu) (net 3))
 (segment (start 176.53 125.095) (end 186.182 125.095) (width 0.25) (layer F.Cu) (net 3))
 (segment (start 175.26 123.825) (end 176.53 125.095) (width 0.25) (layer F.Cu) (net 3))
 (segment (start 187.325 123.952) (end 187.325 122.945) (width 0.25) (layer F.Cu) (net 3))
 (segment (start 175.26 121.92) (end 175.26 123.825) (width 0.25) (layer F.Cu) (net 3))
 (segment (start 180.34 121.92) (end 180.34 116.84) (width 4) (layer B.Cu) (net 2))
 (segment (start 186.7658 110.4142) (end 190.1984 110.4142) (width 4) (layer B.Cu) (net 2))
 (segment (start 180.34 116.84) (end 186.7658 110.4142) (width 4) (layer B.Cu) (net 2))
 (segment (start 174.413 89.9515) (end 189.0115 89.9515) (width 2) (layer B.Cu) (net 2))
 (segment (start 189.0115 89.9515) (end 195.58 96.52) (width 2) (layer B.Cu) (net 2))
 (segment (start 195.58 96.52) (end 195.58 107.95) (width 2) (layer B.Cu) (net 2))
 (segment (start 195.58 107.95) (end 193.04 110.49) (width 2) (layer B.Cu) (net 2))
 (segment (start 192.9642 110.4142) (end 190.1984 110.4142) (width 2) (layer B.Cu) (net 2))
 (segment (start 193.04 110.49) (end 192.9642 110.4142) (width 2) (layer B.Cu) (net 2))
 (segment (start 191.6115 87.3515) (end 189.0115 89.9515) (width 2) (layer B.Cu) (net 2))
 (segment (start 191.6115 74.93) (end 191.6115 87.3515) (width 2) (layer B.Cu) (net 2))
 (segment (start 182.499 121.92) (end 180.34 121.92) (width 0.25) (layer F.Cu) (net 2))
 (segment (start 183.499 122.92) (end 182.499 121.92) (width 0.25) (layer F.Cu) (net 2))
 (segment (start 184.785 122.92) (end 183.499 122.92) (width 0.25) (layer F.Cu) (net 2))
 (segment (start 185.833 69.1515) (end 191.6115 74.93) (width 2) (layer B.Cu) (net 2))
 (segment (start 187.3 120.92) (end 187.325 120.895) (width 0.25) (layer F.Cu) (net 1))
 (segment (start 184.785 120.92) (end 187.3 120.92) (width 0.25) (layer F.Cu) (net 1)))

